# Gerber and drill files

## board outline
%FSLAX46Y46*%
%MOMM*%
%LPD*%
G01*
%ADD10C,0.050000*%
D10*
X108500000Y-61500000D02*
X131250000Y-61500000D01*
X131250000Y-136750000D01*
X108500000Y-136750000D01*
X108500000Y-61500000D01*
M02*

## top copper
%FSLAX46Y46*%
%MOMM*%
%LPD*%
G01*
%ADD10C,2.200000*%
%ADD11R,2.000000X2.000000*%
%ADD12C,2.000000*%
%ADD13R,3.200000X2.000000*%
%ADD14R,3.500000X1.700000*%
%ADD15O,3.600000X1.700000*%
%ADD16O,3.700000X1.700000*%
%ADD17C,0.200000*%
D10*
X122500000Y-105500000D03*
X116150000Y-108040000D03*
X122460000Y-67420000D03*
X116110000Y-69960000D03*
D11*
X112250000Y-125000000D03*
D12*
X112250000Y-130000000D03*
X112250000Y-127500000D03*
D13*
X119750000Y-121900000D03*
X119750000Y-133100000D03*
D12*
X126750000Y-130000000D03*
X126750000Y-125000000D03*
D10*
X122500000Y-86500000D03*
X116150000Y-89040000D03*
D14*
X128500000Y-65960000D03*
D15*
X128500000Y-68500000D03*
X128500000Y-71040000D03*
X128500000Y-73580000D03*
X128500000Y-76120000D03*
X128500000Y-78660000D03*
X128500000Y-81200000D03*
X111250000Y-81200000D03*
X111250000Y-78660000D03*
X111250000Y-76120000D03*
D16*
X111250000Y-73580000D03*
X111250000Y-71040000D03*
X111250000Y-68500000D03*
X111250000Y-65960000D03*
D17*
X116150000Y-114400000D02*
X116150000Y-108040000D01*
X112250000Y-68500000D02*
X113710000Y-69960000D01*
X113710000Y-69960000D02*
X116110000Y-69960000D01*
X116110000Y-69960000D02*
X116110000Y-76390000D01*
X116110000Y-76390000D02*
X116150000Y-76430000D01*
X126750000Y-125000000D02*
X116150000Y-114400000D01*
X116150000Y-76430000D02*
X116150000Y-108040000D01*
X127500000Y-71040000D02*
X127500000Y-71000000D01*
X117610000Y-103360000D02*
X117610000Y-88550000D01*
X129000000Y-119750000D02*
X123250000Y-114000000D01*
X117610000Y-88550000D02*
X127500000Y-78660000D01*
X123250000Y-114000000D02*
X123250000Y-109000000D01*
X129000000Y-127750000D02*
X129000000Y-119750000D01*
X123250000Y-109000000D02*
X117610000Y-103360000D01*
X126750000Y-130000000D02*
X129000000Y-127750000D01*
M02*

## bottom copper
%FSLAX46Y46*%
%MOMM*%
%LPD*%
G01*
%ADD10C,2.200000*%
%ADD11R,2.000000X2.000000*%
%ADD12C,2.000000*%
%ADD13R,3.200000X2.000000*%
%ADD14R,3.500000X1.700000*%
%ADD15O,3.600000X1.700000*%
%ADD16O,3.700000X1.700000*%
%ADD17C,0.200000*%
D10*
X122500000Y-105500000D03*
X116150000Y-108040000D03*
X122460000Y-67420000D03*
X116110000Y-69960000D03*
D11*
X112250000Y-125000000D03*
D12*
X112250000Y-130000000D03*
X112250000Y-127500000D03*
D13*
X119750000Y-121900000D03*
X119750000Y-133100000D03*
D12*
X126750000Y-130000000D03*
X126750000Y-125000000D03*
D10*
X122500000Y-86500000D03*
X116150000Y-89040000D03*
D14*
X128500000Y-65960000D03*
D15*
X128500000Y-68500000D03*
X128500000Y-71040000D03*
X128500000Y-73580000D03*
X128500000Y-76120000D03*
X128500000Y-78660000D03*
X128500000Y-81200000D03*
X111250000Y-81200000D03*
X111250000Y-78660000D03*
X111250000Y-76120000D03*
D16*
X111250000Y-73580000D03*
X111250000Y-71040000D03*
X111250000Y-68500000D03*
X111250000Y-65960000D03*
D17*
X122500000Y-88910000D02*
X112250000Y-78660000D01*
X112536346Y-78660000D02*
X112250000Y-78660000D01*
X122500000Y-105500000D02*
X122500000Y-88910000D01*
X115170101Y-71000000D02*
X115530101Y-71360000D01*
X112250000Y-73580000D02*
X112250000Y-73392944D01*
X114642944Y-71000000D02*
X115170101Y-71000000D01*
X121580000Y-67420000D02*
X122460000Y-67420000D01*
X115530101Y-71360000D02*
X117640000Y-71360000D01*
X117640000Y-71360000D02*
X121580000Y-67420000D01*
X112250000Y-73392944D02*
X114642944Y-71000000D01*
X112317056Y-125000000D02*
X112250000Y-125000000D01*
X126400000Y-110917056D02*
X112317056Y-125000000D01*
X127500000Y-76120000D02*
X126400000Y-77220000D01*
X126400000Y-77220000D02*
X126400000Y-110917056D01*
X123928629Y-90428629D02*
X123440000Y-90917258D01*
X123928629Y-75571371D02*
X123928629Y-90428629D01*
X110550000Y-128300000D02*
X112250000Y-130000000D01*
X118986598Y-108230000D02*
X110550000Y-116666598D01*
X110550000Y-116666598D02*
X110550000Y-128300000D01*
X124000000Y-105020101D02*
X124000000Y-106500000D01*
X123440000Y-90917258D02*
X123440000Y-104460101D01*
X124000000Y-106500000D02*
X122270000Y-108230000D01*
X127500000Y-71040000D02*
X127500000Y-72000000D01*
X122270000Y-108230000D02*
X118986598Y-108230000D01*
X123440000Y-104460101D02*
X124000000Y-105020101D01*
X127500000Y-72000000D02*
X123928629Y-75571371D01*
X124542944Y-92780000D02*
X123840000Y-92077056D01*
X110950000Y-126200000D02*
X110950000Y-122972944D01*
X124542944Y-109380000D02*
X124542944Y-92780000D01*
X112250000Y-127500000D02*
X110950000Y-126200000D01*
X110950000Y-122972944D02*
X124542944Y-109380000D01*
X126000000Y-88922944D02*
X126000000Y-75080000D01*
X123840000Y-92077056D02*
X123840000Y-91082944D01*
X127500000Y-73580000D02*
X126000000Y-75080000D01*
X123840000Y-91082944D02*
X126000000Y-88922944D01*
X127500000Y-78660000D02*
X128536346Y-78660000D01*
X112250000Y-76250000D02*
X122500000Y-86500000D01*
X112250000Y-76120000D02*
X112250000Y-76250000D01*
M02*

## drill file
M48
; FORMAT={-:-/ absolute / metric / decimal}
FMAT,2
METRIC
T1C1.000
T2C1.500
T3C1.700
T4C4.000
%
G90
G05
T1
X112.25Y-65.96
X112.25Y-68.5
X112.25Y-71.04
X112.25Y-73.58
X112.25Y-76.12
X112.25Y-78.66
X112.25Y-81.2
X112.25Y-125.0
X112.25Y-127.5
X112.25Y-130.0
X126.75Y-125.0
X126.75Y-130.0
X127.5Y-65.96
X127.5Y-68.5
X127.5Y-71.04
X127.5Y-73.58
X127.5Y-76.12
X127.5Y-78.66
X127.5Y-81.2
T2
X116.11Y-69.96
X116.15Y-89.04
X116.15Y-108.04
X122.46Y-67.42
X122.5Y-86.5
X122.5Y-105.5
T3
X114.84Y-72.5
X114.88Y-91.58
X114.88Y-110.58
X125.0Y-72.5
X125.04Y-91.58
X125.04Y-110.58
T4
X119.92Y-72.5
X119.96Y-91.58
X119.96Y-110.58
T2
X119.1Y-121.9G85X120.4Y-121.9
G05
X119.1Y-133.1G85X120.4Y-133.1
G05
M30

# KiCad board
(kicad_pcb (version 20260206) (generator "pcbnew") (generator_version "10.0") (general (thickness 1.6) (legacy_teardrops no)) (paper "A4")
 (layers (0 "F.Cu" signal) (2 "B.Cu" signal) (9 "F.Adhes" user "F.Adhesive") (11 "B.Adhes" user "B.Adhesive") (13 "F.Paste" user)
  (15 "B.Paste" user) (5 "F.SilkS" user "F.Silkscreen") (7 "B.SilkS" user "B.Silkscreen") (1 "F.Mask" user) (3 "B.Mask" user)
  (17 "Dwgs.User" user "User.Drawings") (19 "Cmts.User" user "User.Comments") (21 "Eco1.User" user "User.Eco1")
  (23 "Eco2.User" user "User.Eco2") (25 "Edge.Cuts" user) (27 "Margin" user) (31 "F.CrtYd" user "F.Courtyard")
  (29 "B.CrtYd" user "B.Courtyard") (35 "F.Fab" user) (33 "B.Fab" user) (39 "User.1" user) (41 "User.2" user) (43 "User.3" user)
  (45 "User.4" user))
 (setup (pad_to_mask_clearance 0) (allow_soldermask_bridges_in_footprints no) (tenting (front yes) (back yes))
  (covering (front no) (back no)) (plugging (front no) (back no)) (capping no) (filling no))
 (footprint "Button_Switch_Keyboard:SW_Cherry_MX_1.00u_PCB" (layer "F.Cu") (at 122.5 105.5)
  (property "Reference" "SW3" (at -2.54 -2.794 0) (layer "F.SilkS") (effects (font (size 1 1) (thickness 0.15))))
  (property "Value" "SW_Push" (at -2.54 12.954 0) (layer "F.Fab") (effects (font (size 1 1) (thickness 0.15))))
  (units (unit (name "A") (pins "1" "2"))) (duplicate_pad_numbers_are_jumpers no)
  (pad "" np_thru_hole circle (at -7.62 5.08) (size 1.7 1.7) (drill 1.7) (layers "*.Cu" "*.Mask"))
  (pad "" np_thru_hole circle (at -2.54 5.08) (size 4 4) (drill 4) (layers "*.Cu" "*.Mask"))
  (pad "" np_thru_hole circle (at 2.54 5.08) (size 1.7 1.7) (drill 1.7) (layers "*.Cu" "*.Mask"))
  (pad "1" thru_hole circle (at 0 0) (size 2.2 2.2) (drill 1.5) (layers "*.Cu" "*.Mask") (remove_unused_layers no)
   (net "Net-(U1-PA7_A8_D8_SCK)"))
  (pad "2" thru_hole circle (at -6.35 2.54) (size 2.2 2.2) (drill 1.5) (layers "*.Cu" "*.Mask") (remove_unused_layers no) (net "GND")))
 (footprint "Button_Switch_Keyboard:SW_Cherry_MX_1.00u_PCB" (layer "F.Cu") (at 122.46 67.42)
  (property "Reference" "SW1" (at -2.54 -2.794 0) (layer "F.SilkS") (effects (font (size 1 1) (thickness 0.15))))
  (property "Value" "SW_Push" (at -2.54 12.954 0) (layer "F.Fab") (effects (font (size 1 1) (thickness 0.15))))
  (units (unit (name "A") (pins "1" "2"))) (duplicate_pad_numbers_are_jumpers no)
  (pad "" np_thru_hole circle (at -7.62 5.08) (size 1.7 1.7) (drill 1.7) (layers "*.Cu" "*.Mask"))
  (pad "" np_thru_hole circle (at -2.54 5.08) (size 4 4) (drill 4) (layers "*.Cu" "*.Mask"))
  (pad "" np_thru_hole circle (at 2.54 5.08) (size 1.7 1.7) (drill 1.7) (layers "*.Cu" "*.Mask"))
  (pad "1" thru_hole circle (at 0 0) (size 2.2 2.2) (drill 1.5) (layers "*.Cu" "*.Mask") (remove_unused_layers no)
   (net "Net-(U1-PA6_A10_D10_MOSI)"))
  (pad "2" thru_hole circle (at -6.35 2.54) (size 2.2 2.2) (drill 1.5) (layers "*.Cu" "*.Mask") (remove_unused_layers no) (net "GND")))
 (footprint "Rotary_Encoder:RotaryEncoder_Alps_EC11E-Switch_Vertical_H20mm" (layer "F.Cu") (at 112.25 125)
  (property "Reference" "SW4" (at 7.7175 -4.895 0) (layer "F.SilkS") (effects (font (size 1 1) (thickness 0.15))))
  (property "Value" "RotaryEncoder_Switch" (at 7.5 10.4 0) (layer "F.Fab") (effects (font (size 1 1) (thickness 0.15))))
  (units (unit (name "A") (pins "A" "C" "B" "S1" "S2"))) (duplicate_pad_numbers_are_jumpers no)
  (pad "A" thru_hole rect (at 0 0) (size 2 2) (drill 1) (layers "*.Cu" "*.Mask") (remove_unused_layers no) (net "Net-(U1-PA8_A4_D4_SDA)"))
  (pad "B" thru_hole circle (at 0 5) (size 2 2) (drill 1) (layers "*.Cu" "*.Mask") (remove_unused_layers no) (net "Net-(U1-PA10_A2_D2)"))
  (pad "C" thru_hole circle (at 0 2.5) (size 2 2) (drill 1) (layers "*.Cu" "*.Mask") (remove_unused_layers no) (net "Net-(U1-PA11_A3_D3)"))
  (pad "MP" thru_hole rect (at 7.5 -3.1) (size 3.2 2) (drill oval 2.8 1.5) (layers "*.Cu" "*.Mask") (remove_unused_layers no))
  (pad "MP" thru_hole rect (at 7.5 8.1) (size 3.2 2) (drill oval 2.8 1.5) (layers "*.Cu" "*.Mask") (remove_unused_layers no))
  (pad "S1" thru_hole circle (at 14.5 5) (size 2 2) (drill 1) (layers "*.Cu" "*.Mask") (remove_unused_layers no)
   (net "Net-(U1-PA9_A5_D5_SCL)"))
  (pad "S2" thru_hole circle (at 14.5 0) (size 2 2) (drill 1) (layers "*.Cu" "*.Mask") (remove_unused_layers no) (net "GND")))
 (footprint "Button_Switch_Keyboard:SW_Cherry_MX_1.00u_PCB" (layer "F.Cu") (at 122.5 86.5)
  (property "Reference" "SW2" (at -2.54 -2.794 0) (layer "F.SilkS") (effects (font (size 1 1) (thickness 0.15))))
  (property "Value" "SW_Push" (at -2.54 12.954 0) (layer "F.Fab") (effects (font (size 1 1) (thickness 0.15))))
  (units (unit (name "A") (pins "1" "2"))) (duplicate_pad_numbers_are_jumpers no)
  (pad "" np_thru_hole circle (at -7.62 5.08) (size 1.7 1.7) (drill 1.7) (layers "*.Cu" "*.Mask"))
  (pad "" np_thru_hole circle (at -2.54 5.08) (size 4 4) (drill 4) (layers "*.Cu" "*.Mask"))
  (pad "" np_thru_hole circle (at 2.54 5.08) (size 1.7 1.7) (drill 1.7) (layers "*.Cu" "*.Mask"))
  (pad "1" thru_hole circle (at 0 0) (size 2.2 2.2) (drill 1.5) (layers "*.Cu" "*.Mask") (remove_unused_layers no)
   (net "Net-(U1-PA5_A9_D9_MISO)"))
  (pad "2" thru_hole circle (at -6.35 2.54) (size 2.2 2.2) (drill 1.5) (layers "*.Cu" "*.Mask") (remove_unused_layers no) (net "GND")))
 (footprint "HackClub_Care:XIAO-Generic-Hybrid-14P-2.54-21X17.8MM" (layer "B.Cu") (at 119.875 73.58 180)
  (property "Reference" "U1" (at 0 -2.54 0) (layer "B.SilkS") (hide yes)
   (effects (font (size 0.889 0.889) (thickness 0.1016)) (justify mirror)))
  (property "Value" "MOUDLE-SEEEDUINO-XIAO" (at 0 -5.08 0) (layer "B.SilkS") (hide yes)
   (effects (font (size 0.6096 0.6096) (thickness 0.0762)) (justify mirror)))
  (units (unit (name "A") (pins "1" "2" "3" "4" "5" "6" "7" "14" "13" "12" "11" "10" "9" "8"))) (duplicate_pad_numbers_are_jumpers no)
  (pad "1" thru_hole rect (at -7.625 7.62 180) (size 3.5 1.7) (drill 1 (offset -1 0)) (layers "*.Cu" "*.Mask") (remove_unused_layers no)
   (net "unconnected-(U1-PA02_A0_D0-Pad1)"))
  (pad "2" thru_hole oval (at -7.625 5.08 180) (size 3.6 1.7) (drill 1 (offset -1 0)) (layers "*.Cu" "*.Mask") (remove_unused_layers no)
   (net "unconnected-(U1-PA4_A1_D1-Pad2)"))
  (pad "3" thru_hole oval (at -7.625 2.54 180) (size 3.6 1.7) (drill 1 (offset -1 0)) (layers "*.Cu" "*.Mask") (remove_unused_layers no)
   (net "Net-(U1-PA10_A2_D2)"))
  (pad "4" thru_hole oval (at -7.625 0 180) (size 3.6 1.7) (drill 1 (offset -1 0)) (layers "*.Cu" "*.Mask") (remove_unused_layers no)
   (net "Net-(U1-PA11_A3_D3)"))
  (pad "5" thru_hole oval (at -7.625 -2.54 180) (size 3.6 1.7) (drill 1 (offset -1 0)) (layers "*.Cu" "*.Mask") (remove_unused_layers no)
   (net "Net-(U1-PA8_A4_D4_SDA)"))
  (pad "6" thru_hole oval (at -7.625 -5.08) (size 3.6 1.7) (drill 1 (offset 1 0)) (layers "*.Cu" "*.Mask") (remove_unused_layers no)
   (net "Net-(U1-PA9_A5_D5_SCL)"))
  (pad "7" thru_hole oval (at -7.625 -7.62 180) (size 3.6 1.7) (drill 1 (offset -1 0)) (layers "*.Cu" "*.Mask") (remove_unused_layers no)
   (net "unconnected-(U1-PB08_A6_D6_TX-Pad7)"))
  (pad "8" thru_hole oval (at 7.625 -7.62 180) (size 3.6 1.7) (drill 1 (offset 1 0)) (layers "*.Cu" "*.Mask") (remove_unused_layers no)
   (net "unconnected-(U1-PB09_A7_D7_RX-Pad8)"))
  (pad "9" thru_hole oval (at 7.625 -5.08 180) (size 3.6 1.7) (drill 1 (offset 1 0)) (layers "*.Cu" "*.Mask") (remove_unused_layers no)
   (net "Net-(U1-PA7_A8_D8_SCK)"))
  (pad "10" thru_hole oval (at 7.625 -2.54 180) (size 3.6 1.7) (drill 1 (offset 1 0)) (layers "*.Cu" "*.Mask") (remove_unused_layers no)
   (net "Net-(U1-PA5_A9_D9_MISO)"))
  (pad "11" thru_hole oval (at 7.625 0 180) (size 3.7 1.7) (drill 1 (offset 1 0)) (layers "*.Cu" "*.Mask") (remove_unused_layers no)
   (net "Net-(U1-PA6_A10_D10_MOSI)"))
  (pad "12" thru_hole oval (at 7.625 2.54 180) (size 3.7 1.7) (drill 1 (offset 1 0)) (layers "*.Cu" "*.Mask") (remove_unused_layers no)
   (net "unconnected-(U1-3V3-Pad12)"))
  (pad "13" thru_hole oval (at 7.625 5.08 180) (size 3.7 1.7) (drill 1 (offset 1 0)) (layers "*.Cu" "*.Mask") (remove_unused_layers no)
   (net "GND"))
  (pad "14" thru_hole oval (at 7.625 7.62 180) (size 3.7 1.7) (drill 1 (offset 1 0)) (layers "*.Cu" "*.Mask") (remove_unused_layers no)
   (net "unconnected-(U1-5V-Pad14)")))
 (gr_rect (start 108.5 61.5) (end 131.25 136.75) (stroke (width 0.05) (type default)) (fill no) (layer "Edge.Cuts"))
 (segment (start 122.5 88.91) (end 112.25 78.66) (width 0.2) (layer "B.Cu") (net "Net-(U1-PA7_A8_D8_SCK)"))
 (segment (start 112.536346 78.66) (end 112.25 78.66) (width 0.2) (layer "B.Cu") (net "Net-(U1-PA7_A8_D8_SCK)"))
 (segment (start 122.5 105.5) (end 122.5 88.91) (width 0.2) (layer "B.Cu") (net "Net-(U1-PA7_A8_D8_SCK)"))
 (segment (start 116.15 114.4) (end 116.15 108.04) (width 0.2) (layer "F.Cu") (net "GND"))
 (segment (start 112.25 68.5) (end 113.71 69.96) (width 0.2) (layer "F.Cu") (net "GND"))
 (segment (start 113.71 69.96) (end 116.11 69.96) (width 0.2) (layer "F.Cu") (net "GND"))
 (segment (start 116.11 69.96) (end 116.11 76.39) (width 0.2) (layer "F.Cu") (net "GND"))
 (segment (start 116.11 76.39) (end 116.15 76.43) (width 0.2) (layer "F.Cu") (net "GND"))
 (segment (start 126.75 125) (end 116.15 114.4) (width 0.2) (layer "F.Cu") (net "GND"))
 (segment (start 116.15 76.43) (end 116.15 108.04) (width 0.2) (layer "F.Cu") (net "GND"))
 (segment (start 115.170101 71) (end 115.530101 71.36) (width 0.2) (layer "B.Cu") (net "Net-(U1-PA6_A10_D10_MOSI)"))
 (segment (start 112.25 73.58) (end 112.25 73.392944) (width 0.2) (layer "B.Cu") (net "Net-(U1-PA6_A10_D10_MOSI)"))
 (segment (start 114.642944 71) (end 115.170101 71) (width 0.2) (layer "B.Cu") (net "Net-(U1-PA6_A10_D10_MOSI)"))
 (segment (start 121.58 67.42) (end 122.46 67.42) (width 0.2) (layer "B.Cu") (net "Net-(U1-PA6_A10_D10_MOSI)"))
 (segment (start 115.530101 71.36) (end 117.64 71.36) (width 0.2) (layer "B.Cu") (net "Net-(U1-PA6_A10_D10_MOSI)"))
 (segment (start 117.64 71.36) (end 121.58 67.42) (width 0.2) (layer "B.Cu") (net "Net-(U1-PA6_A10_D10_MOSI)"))
 (segment (start 112.25 73.392944) (end 114.642944 71) (width 0.2) (layer "B.Cu") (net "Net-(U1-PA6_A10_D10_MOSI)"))
 (segment (start 112.317056 125) (end 112.25 125) (width 0.2) (layer "B.Cu") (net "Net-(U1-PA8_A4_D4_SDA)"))
 (segment (start 126.4 110.917056) (end 112.317056 125) (width 0.2) (layer "B.Cu") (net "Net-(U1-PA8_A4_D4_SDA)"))
 (segment (start 127.5 76.12) (end 126.4 77.22) (width 0.2) (layer "B.Cu") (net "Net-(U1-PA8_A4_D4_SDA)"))
 (segment (start 126.4 77.22) (end 126.4 110.917056) (width 0.2) (layer "B.Cu") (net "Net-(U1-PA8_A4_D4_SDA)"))
 (segment (start 127.5 71.04) (end 127.5 71) (width 0.2) (layer "F.Cu") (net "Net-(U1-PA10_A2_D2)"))
 (segment (start 123.928629 90.428629) (end 123.44 90.917258) (width 0.2) (layer "B.Cu") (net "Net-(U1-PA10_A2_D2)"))
 (segment (start 123.928629 75.571371) (end 123.928629 90.428629) (width 0.2) (layer "B.Cu") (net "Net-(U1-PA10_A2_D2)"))
 (segment (start 110.55 128.3) (end 112.25 130) (width 0.2) (layer "B.Cu") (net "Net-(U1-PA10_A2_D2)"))
 (segment (start 118.986598 108.23) (end 110.55 116.666598) (width 0.2) (layer "B.Cu") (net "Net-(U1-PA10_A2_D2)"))
 (segment (start 110.55 116.666598) (end 110.55 128.3) (width 0.2) (layer "B.Cu") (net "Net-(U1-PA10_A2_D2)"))
 (segment (start 124 105.020101) (end 124 106.5) (width 0.2) (layer "B.Cu") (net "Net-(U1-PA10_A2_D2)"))
 (segment (start 123.44 90.917258) (end 123.44 104.460101) (width 0.2) (layer "B.Cu") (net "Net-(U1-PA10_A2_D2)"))
 (segment (start 124 106.5) (end 122.27 108.23) (width 0.2) (layer "B.Cu") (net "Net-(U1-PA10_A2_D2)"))
 (segment (start 127.5 71.04) (end 127.5 72) (width 0.2) (layer "B.Cu") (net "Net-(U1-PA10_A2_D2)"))
 (segment (start 122.27 108.23) (end 118.986598 108.23) (width 0.2) (layer "B.Cu") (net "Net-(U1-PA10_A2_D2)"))
 (segment (start 123.44 104.460101) (end 124 105.020101) (width 0.2) (layer "B.Cu") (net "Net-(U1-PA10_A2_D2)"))
 (segment (start 127.5 72) (end 123.928629 75.571371) (width 0.2) (layer "B.Cu") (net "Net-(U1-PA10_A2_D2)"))
 (segment (start 124.542944 92.78) (end 123.84 92.077056) (width 0.2) (layer "B.Cu") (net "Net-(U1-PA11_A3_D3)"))
 (segment (start 110.95 126.2) (end 110.95 122.972944) (width 0.2) (layer "B.Cu") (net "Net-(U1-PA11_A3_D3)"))
 (segment (start 124.542944 109.38) (end 124.542944 92.78) (width 0.2) (layer "B.Cu") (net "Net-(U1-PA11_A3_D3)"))
 (segment (start 112.25 127.5) (end 110.95 126.2) (width 0.2) (layer "B.Cu") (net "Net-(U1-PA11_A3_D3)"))
 (segment (start 110.95 122.972944) (end 124.542944 109.38) (width 0.2) (layer "B.Cu") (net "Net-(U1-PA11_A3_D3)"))
 (segment (start 126 88.922944) (end 126 75.08) (width 0.2) (layer "B.Cu") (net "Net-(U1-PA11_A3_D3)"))
 (segment (start 123.84 92.077056) (end 123.84 91.082944) (width 0.2) (layer "B.Cu") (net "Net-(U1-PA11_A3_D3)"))
 (segment (start 127.5 73.58) (end 126 75.08) (width 0.2) (layer "B.Cu") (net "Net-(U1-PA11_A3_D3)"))
 (segment (start 123.84 91.082944) (end 126 88.922944) (width 0.2) (layer "B.Cu") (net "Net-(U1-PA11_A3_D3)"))
 (segment (start 117.61 103.36) (end 117.61 88.55) (width 0.2) (layer "F.Cu") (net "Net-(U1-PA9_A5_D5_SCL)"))
 (segment (start 129 119.75) (end 123.25 114) (width 0.2) (layer "F.Cu") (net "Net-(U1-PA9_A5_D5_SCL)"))
 (segment (start 117.61 88.55) (end 127.5 78.66) (width 0.2) (layer "F.Cu") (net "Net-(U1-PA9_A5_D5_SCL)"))
 (segment (start 123.25 114) (end 123.25 109) (width 0.2) (layer "F.Cu") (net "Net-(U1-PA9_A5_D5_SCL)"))
 (segment (start 129 127.75) (end 129 119.75) (width 0.2) (layer "F.Cu") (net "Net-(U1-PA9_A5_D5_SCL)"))
 (segment (start 123.25 109) (end 117.61 103.36) (width 0.2) (layer "F.Cu") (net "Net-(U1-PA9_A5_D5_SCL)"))
 (segment (start 126.75 130) (end 129 127.75) (width 0.2) (layer "F.Cu") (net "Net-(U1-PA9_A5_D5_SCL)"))
 (segment (start 127.5 78.66) (end 128.536346 78.66) (width 0.2) (layer "B.Cu") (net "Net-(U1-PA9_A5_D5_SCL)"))
 (segment (start 112.25 76.25) (end 122.5 86.5) (width 0.2) (layer "B.Cu") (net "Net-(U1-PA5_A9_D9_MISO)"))
 (segment (start 112.25 76.12) (end 112.25 76.25) (width 0.2) (layer "B.Cu") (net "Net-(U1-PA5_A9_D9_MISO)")))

